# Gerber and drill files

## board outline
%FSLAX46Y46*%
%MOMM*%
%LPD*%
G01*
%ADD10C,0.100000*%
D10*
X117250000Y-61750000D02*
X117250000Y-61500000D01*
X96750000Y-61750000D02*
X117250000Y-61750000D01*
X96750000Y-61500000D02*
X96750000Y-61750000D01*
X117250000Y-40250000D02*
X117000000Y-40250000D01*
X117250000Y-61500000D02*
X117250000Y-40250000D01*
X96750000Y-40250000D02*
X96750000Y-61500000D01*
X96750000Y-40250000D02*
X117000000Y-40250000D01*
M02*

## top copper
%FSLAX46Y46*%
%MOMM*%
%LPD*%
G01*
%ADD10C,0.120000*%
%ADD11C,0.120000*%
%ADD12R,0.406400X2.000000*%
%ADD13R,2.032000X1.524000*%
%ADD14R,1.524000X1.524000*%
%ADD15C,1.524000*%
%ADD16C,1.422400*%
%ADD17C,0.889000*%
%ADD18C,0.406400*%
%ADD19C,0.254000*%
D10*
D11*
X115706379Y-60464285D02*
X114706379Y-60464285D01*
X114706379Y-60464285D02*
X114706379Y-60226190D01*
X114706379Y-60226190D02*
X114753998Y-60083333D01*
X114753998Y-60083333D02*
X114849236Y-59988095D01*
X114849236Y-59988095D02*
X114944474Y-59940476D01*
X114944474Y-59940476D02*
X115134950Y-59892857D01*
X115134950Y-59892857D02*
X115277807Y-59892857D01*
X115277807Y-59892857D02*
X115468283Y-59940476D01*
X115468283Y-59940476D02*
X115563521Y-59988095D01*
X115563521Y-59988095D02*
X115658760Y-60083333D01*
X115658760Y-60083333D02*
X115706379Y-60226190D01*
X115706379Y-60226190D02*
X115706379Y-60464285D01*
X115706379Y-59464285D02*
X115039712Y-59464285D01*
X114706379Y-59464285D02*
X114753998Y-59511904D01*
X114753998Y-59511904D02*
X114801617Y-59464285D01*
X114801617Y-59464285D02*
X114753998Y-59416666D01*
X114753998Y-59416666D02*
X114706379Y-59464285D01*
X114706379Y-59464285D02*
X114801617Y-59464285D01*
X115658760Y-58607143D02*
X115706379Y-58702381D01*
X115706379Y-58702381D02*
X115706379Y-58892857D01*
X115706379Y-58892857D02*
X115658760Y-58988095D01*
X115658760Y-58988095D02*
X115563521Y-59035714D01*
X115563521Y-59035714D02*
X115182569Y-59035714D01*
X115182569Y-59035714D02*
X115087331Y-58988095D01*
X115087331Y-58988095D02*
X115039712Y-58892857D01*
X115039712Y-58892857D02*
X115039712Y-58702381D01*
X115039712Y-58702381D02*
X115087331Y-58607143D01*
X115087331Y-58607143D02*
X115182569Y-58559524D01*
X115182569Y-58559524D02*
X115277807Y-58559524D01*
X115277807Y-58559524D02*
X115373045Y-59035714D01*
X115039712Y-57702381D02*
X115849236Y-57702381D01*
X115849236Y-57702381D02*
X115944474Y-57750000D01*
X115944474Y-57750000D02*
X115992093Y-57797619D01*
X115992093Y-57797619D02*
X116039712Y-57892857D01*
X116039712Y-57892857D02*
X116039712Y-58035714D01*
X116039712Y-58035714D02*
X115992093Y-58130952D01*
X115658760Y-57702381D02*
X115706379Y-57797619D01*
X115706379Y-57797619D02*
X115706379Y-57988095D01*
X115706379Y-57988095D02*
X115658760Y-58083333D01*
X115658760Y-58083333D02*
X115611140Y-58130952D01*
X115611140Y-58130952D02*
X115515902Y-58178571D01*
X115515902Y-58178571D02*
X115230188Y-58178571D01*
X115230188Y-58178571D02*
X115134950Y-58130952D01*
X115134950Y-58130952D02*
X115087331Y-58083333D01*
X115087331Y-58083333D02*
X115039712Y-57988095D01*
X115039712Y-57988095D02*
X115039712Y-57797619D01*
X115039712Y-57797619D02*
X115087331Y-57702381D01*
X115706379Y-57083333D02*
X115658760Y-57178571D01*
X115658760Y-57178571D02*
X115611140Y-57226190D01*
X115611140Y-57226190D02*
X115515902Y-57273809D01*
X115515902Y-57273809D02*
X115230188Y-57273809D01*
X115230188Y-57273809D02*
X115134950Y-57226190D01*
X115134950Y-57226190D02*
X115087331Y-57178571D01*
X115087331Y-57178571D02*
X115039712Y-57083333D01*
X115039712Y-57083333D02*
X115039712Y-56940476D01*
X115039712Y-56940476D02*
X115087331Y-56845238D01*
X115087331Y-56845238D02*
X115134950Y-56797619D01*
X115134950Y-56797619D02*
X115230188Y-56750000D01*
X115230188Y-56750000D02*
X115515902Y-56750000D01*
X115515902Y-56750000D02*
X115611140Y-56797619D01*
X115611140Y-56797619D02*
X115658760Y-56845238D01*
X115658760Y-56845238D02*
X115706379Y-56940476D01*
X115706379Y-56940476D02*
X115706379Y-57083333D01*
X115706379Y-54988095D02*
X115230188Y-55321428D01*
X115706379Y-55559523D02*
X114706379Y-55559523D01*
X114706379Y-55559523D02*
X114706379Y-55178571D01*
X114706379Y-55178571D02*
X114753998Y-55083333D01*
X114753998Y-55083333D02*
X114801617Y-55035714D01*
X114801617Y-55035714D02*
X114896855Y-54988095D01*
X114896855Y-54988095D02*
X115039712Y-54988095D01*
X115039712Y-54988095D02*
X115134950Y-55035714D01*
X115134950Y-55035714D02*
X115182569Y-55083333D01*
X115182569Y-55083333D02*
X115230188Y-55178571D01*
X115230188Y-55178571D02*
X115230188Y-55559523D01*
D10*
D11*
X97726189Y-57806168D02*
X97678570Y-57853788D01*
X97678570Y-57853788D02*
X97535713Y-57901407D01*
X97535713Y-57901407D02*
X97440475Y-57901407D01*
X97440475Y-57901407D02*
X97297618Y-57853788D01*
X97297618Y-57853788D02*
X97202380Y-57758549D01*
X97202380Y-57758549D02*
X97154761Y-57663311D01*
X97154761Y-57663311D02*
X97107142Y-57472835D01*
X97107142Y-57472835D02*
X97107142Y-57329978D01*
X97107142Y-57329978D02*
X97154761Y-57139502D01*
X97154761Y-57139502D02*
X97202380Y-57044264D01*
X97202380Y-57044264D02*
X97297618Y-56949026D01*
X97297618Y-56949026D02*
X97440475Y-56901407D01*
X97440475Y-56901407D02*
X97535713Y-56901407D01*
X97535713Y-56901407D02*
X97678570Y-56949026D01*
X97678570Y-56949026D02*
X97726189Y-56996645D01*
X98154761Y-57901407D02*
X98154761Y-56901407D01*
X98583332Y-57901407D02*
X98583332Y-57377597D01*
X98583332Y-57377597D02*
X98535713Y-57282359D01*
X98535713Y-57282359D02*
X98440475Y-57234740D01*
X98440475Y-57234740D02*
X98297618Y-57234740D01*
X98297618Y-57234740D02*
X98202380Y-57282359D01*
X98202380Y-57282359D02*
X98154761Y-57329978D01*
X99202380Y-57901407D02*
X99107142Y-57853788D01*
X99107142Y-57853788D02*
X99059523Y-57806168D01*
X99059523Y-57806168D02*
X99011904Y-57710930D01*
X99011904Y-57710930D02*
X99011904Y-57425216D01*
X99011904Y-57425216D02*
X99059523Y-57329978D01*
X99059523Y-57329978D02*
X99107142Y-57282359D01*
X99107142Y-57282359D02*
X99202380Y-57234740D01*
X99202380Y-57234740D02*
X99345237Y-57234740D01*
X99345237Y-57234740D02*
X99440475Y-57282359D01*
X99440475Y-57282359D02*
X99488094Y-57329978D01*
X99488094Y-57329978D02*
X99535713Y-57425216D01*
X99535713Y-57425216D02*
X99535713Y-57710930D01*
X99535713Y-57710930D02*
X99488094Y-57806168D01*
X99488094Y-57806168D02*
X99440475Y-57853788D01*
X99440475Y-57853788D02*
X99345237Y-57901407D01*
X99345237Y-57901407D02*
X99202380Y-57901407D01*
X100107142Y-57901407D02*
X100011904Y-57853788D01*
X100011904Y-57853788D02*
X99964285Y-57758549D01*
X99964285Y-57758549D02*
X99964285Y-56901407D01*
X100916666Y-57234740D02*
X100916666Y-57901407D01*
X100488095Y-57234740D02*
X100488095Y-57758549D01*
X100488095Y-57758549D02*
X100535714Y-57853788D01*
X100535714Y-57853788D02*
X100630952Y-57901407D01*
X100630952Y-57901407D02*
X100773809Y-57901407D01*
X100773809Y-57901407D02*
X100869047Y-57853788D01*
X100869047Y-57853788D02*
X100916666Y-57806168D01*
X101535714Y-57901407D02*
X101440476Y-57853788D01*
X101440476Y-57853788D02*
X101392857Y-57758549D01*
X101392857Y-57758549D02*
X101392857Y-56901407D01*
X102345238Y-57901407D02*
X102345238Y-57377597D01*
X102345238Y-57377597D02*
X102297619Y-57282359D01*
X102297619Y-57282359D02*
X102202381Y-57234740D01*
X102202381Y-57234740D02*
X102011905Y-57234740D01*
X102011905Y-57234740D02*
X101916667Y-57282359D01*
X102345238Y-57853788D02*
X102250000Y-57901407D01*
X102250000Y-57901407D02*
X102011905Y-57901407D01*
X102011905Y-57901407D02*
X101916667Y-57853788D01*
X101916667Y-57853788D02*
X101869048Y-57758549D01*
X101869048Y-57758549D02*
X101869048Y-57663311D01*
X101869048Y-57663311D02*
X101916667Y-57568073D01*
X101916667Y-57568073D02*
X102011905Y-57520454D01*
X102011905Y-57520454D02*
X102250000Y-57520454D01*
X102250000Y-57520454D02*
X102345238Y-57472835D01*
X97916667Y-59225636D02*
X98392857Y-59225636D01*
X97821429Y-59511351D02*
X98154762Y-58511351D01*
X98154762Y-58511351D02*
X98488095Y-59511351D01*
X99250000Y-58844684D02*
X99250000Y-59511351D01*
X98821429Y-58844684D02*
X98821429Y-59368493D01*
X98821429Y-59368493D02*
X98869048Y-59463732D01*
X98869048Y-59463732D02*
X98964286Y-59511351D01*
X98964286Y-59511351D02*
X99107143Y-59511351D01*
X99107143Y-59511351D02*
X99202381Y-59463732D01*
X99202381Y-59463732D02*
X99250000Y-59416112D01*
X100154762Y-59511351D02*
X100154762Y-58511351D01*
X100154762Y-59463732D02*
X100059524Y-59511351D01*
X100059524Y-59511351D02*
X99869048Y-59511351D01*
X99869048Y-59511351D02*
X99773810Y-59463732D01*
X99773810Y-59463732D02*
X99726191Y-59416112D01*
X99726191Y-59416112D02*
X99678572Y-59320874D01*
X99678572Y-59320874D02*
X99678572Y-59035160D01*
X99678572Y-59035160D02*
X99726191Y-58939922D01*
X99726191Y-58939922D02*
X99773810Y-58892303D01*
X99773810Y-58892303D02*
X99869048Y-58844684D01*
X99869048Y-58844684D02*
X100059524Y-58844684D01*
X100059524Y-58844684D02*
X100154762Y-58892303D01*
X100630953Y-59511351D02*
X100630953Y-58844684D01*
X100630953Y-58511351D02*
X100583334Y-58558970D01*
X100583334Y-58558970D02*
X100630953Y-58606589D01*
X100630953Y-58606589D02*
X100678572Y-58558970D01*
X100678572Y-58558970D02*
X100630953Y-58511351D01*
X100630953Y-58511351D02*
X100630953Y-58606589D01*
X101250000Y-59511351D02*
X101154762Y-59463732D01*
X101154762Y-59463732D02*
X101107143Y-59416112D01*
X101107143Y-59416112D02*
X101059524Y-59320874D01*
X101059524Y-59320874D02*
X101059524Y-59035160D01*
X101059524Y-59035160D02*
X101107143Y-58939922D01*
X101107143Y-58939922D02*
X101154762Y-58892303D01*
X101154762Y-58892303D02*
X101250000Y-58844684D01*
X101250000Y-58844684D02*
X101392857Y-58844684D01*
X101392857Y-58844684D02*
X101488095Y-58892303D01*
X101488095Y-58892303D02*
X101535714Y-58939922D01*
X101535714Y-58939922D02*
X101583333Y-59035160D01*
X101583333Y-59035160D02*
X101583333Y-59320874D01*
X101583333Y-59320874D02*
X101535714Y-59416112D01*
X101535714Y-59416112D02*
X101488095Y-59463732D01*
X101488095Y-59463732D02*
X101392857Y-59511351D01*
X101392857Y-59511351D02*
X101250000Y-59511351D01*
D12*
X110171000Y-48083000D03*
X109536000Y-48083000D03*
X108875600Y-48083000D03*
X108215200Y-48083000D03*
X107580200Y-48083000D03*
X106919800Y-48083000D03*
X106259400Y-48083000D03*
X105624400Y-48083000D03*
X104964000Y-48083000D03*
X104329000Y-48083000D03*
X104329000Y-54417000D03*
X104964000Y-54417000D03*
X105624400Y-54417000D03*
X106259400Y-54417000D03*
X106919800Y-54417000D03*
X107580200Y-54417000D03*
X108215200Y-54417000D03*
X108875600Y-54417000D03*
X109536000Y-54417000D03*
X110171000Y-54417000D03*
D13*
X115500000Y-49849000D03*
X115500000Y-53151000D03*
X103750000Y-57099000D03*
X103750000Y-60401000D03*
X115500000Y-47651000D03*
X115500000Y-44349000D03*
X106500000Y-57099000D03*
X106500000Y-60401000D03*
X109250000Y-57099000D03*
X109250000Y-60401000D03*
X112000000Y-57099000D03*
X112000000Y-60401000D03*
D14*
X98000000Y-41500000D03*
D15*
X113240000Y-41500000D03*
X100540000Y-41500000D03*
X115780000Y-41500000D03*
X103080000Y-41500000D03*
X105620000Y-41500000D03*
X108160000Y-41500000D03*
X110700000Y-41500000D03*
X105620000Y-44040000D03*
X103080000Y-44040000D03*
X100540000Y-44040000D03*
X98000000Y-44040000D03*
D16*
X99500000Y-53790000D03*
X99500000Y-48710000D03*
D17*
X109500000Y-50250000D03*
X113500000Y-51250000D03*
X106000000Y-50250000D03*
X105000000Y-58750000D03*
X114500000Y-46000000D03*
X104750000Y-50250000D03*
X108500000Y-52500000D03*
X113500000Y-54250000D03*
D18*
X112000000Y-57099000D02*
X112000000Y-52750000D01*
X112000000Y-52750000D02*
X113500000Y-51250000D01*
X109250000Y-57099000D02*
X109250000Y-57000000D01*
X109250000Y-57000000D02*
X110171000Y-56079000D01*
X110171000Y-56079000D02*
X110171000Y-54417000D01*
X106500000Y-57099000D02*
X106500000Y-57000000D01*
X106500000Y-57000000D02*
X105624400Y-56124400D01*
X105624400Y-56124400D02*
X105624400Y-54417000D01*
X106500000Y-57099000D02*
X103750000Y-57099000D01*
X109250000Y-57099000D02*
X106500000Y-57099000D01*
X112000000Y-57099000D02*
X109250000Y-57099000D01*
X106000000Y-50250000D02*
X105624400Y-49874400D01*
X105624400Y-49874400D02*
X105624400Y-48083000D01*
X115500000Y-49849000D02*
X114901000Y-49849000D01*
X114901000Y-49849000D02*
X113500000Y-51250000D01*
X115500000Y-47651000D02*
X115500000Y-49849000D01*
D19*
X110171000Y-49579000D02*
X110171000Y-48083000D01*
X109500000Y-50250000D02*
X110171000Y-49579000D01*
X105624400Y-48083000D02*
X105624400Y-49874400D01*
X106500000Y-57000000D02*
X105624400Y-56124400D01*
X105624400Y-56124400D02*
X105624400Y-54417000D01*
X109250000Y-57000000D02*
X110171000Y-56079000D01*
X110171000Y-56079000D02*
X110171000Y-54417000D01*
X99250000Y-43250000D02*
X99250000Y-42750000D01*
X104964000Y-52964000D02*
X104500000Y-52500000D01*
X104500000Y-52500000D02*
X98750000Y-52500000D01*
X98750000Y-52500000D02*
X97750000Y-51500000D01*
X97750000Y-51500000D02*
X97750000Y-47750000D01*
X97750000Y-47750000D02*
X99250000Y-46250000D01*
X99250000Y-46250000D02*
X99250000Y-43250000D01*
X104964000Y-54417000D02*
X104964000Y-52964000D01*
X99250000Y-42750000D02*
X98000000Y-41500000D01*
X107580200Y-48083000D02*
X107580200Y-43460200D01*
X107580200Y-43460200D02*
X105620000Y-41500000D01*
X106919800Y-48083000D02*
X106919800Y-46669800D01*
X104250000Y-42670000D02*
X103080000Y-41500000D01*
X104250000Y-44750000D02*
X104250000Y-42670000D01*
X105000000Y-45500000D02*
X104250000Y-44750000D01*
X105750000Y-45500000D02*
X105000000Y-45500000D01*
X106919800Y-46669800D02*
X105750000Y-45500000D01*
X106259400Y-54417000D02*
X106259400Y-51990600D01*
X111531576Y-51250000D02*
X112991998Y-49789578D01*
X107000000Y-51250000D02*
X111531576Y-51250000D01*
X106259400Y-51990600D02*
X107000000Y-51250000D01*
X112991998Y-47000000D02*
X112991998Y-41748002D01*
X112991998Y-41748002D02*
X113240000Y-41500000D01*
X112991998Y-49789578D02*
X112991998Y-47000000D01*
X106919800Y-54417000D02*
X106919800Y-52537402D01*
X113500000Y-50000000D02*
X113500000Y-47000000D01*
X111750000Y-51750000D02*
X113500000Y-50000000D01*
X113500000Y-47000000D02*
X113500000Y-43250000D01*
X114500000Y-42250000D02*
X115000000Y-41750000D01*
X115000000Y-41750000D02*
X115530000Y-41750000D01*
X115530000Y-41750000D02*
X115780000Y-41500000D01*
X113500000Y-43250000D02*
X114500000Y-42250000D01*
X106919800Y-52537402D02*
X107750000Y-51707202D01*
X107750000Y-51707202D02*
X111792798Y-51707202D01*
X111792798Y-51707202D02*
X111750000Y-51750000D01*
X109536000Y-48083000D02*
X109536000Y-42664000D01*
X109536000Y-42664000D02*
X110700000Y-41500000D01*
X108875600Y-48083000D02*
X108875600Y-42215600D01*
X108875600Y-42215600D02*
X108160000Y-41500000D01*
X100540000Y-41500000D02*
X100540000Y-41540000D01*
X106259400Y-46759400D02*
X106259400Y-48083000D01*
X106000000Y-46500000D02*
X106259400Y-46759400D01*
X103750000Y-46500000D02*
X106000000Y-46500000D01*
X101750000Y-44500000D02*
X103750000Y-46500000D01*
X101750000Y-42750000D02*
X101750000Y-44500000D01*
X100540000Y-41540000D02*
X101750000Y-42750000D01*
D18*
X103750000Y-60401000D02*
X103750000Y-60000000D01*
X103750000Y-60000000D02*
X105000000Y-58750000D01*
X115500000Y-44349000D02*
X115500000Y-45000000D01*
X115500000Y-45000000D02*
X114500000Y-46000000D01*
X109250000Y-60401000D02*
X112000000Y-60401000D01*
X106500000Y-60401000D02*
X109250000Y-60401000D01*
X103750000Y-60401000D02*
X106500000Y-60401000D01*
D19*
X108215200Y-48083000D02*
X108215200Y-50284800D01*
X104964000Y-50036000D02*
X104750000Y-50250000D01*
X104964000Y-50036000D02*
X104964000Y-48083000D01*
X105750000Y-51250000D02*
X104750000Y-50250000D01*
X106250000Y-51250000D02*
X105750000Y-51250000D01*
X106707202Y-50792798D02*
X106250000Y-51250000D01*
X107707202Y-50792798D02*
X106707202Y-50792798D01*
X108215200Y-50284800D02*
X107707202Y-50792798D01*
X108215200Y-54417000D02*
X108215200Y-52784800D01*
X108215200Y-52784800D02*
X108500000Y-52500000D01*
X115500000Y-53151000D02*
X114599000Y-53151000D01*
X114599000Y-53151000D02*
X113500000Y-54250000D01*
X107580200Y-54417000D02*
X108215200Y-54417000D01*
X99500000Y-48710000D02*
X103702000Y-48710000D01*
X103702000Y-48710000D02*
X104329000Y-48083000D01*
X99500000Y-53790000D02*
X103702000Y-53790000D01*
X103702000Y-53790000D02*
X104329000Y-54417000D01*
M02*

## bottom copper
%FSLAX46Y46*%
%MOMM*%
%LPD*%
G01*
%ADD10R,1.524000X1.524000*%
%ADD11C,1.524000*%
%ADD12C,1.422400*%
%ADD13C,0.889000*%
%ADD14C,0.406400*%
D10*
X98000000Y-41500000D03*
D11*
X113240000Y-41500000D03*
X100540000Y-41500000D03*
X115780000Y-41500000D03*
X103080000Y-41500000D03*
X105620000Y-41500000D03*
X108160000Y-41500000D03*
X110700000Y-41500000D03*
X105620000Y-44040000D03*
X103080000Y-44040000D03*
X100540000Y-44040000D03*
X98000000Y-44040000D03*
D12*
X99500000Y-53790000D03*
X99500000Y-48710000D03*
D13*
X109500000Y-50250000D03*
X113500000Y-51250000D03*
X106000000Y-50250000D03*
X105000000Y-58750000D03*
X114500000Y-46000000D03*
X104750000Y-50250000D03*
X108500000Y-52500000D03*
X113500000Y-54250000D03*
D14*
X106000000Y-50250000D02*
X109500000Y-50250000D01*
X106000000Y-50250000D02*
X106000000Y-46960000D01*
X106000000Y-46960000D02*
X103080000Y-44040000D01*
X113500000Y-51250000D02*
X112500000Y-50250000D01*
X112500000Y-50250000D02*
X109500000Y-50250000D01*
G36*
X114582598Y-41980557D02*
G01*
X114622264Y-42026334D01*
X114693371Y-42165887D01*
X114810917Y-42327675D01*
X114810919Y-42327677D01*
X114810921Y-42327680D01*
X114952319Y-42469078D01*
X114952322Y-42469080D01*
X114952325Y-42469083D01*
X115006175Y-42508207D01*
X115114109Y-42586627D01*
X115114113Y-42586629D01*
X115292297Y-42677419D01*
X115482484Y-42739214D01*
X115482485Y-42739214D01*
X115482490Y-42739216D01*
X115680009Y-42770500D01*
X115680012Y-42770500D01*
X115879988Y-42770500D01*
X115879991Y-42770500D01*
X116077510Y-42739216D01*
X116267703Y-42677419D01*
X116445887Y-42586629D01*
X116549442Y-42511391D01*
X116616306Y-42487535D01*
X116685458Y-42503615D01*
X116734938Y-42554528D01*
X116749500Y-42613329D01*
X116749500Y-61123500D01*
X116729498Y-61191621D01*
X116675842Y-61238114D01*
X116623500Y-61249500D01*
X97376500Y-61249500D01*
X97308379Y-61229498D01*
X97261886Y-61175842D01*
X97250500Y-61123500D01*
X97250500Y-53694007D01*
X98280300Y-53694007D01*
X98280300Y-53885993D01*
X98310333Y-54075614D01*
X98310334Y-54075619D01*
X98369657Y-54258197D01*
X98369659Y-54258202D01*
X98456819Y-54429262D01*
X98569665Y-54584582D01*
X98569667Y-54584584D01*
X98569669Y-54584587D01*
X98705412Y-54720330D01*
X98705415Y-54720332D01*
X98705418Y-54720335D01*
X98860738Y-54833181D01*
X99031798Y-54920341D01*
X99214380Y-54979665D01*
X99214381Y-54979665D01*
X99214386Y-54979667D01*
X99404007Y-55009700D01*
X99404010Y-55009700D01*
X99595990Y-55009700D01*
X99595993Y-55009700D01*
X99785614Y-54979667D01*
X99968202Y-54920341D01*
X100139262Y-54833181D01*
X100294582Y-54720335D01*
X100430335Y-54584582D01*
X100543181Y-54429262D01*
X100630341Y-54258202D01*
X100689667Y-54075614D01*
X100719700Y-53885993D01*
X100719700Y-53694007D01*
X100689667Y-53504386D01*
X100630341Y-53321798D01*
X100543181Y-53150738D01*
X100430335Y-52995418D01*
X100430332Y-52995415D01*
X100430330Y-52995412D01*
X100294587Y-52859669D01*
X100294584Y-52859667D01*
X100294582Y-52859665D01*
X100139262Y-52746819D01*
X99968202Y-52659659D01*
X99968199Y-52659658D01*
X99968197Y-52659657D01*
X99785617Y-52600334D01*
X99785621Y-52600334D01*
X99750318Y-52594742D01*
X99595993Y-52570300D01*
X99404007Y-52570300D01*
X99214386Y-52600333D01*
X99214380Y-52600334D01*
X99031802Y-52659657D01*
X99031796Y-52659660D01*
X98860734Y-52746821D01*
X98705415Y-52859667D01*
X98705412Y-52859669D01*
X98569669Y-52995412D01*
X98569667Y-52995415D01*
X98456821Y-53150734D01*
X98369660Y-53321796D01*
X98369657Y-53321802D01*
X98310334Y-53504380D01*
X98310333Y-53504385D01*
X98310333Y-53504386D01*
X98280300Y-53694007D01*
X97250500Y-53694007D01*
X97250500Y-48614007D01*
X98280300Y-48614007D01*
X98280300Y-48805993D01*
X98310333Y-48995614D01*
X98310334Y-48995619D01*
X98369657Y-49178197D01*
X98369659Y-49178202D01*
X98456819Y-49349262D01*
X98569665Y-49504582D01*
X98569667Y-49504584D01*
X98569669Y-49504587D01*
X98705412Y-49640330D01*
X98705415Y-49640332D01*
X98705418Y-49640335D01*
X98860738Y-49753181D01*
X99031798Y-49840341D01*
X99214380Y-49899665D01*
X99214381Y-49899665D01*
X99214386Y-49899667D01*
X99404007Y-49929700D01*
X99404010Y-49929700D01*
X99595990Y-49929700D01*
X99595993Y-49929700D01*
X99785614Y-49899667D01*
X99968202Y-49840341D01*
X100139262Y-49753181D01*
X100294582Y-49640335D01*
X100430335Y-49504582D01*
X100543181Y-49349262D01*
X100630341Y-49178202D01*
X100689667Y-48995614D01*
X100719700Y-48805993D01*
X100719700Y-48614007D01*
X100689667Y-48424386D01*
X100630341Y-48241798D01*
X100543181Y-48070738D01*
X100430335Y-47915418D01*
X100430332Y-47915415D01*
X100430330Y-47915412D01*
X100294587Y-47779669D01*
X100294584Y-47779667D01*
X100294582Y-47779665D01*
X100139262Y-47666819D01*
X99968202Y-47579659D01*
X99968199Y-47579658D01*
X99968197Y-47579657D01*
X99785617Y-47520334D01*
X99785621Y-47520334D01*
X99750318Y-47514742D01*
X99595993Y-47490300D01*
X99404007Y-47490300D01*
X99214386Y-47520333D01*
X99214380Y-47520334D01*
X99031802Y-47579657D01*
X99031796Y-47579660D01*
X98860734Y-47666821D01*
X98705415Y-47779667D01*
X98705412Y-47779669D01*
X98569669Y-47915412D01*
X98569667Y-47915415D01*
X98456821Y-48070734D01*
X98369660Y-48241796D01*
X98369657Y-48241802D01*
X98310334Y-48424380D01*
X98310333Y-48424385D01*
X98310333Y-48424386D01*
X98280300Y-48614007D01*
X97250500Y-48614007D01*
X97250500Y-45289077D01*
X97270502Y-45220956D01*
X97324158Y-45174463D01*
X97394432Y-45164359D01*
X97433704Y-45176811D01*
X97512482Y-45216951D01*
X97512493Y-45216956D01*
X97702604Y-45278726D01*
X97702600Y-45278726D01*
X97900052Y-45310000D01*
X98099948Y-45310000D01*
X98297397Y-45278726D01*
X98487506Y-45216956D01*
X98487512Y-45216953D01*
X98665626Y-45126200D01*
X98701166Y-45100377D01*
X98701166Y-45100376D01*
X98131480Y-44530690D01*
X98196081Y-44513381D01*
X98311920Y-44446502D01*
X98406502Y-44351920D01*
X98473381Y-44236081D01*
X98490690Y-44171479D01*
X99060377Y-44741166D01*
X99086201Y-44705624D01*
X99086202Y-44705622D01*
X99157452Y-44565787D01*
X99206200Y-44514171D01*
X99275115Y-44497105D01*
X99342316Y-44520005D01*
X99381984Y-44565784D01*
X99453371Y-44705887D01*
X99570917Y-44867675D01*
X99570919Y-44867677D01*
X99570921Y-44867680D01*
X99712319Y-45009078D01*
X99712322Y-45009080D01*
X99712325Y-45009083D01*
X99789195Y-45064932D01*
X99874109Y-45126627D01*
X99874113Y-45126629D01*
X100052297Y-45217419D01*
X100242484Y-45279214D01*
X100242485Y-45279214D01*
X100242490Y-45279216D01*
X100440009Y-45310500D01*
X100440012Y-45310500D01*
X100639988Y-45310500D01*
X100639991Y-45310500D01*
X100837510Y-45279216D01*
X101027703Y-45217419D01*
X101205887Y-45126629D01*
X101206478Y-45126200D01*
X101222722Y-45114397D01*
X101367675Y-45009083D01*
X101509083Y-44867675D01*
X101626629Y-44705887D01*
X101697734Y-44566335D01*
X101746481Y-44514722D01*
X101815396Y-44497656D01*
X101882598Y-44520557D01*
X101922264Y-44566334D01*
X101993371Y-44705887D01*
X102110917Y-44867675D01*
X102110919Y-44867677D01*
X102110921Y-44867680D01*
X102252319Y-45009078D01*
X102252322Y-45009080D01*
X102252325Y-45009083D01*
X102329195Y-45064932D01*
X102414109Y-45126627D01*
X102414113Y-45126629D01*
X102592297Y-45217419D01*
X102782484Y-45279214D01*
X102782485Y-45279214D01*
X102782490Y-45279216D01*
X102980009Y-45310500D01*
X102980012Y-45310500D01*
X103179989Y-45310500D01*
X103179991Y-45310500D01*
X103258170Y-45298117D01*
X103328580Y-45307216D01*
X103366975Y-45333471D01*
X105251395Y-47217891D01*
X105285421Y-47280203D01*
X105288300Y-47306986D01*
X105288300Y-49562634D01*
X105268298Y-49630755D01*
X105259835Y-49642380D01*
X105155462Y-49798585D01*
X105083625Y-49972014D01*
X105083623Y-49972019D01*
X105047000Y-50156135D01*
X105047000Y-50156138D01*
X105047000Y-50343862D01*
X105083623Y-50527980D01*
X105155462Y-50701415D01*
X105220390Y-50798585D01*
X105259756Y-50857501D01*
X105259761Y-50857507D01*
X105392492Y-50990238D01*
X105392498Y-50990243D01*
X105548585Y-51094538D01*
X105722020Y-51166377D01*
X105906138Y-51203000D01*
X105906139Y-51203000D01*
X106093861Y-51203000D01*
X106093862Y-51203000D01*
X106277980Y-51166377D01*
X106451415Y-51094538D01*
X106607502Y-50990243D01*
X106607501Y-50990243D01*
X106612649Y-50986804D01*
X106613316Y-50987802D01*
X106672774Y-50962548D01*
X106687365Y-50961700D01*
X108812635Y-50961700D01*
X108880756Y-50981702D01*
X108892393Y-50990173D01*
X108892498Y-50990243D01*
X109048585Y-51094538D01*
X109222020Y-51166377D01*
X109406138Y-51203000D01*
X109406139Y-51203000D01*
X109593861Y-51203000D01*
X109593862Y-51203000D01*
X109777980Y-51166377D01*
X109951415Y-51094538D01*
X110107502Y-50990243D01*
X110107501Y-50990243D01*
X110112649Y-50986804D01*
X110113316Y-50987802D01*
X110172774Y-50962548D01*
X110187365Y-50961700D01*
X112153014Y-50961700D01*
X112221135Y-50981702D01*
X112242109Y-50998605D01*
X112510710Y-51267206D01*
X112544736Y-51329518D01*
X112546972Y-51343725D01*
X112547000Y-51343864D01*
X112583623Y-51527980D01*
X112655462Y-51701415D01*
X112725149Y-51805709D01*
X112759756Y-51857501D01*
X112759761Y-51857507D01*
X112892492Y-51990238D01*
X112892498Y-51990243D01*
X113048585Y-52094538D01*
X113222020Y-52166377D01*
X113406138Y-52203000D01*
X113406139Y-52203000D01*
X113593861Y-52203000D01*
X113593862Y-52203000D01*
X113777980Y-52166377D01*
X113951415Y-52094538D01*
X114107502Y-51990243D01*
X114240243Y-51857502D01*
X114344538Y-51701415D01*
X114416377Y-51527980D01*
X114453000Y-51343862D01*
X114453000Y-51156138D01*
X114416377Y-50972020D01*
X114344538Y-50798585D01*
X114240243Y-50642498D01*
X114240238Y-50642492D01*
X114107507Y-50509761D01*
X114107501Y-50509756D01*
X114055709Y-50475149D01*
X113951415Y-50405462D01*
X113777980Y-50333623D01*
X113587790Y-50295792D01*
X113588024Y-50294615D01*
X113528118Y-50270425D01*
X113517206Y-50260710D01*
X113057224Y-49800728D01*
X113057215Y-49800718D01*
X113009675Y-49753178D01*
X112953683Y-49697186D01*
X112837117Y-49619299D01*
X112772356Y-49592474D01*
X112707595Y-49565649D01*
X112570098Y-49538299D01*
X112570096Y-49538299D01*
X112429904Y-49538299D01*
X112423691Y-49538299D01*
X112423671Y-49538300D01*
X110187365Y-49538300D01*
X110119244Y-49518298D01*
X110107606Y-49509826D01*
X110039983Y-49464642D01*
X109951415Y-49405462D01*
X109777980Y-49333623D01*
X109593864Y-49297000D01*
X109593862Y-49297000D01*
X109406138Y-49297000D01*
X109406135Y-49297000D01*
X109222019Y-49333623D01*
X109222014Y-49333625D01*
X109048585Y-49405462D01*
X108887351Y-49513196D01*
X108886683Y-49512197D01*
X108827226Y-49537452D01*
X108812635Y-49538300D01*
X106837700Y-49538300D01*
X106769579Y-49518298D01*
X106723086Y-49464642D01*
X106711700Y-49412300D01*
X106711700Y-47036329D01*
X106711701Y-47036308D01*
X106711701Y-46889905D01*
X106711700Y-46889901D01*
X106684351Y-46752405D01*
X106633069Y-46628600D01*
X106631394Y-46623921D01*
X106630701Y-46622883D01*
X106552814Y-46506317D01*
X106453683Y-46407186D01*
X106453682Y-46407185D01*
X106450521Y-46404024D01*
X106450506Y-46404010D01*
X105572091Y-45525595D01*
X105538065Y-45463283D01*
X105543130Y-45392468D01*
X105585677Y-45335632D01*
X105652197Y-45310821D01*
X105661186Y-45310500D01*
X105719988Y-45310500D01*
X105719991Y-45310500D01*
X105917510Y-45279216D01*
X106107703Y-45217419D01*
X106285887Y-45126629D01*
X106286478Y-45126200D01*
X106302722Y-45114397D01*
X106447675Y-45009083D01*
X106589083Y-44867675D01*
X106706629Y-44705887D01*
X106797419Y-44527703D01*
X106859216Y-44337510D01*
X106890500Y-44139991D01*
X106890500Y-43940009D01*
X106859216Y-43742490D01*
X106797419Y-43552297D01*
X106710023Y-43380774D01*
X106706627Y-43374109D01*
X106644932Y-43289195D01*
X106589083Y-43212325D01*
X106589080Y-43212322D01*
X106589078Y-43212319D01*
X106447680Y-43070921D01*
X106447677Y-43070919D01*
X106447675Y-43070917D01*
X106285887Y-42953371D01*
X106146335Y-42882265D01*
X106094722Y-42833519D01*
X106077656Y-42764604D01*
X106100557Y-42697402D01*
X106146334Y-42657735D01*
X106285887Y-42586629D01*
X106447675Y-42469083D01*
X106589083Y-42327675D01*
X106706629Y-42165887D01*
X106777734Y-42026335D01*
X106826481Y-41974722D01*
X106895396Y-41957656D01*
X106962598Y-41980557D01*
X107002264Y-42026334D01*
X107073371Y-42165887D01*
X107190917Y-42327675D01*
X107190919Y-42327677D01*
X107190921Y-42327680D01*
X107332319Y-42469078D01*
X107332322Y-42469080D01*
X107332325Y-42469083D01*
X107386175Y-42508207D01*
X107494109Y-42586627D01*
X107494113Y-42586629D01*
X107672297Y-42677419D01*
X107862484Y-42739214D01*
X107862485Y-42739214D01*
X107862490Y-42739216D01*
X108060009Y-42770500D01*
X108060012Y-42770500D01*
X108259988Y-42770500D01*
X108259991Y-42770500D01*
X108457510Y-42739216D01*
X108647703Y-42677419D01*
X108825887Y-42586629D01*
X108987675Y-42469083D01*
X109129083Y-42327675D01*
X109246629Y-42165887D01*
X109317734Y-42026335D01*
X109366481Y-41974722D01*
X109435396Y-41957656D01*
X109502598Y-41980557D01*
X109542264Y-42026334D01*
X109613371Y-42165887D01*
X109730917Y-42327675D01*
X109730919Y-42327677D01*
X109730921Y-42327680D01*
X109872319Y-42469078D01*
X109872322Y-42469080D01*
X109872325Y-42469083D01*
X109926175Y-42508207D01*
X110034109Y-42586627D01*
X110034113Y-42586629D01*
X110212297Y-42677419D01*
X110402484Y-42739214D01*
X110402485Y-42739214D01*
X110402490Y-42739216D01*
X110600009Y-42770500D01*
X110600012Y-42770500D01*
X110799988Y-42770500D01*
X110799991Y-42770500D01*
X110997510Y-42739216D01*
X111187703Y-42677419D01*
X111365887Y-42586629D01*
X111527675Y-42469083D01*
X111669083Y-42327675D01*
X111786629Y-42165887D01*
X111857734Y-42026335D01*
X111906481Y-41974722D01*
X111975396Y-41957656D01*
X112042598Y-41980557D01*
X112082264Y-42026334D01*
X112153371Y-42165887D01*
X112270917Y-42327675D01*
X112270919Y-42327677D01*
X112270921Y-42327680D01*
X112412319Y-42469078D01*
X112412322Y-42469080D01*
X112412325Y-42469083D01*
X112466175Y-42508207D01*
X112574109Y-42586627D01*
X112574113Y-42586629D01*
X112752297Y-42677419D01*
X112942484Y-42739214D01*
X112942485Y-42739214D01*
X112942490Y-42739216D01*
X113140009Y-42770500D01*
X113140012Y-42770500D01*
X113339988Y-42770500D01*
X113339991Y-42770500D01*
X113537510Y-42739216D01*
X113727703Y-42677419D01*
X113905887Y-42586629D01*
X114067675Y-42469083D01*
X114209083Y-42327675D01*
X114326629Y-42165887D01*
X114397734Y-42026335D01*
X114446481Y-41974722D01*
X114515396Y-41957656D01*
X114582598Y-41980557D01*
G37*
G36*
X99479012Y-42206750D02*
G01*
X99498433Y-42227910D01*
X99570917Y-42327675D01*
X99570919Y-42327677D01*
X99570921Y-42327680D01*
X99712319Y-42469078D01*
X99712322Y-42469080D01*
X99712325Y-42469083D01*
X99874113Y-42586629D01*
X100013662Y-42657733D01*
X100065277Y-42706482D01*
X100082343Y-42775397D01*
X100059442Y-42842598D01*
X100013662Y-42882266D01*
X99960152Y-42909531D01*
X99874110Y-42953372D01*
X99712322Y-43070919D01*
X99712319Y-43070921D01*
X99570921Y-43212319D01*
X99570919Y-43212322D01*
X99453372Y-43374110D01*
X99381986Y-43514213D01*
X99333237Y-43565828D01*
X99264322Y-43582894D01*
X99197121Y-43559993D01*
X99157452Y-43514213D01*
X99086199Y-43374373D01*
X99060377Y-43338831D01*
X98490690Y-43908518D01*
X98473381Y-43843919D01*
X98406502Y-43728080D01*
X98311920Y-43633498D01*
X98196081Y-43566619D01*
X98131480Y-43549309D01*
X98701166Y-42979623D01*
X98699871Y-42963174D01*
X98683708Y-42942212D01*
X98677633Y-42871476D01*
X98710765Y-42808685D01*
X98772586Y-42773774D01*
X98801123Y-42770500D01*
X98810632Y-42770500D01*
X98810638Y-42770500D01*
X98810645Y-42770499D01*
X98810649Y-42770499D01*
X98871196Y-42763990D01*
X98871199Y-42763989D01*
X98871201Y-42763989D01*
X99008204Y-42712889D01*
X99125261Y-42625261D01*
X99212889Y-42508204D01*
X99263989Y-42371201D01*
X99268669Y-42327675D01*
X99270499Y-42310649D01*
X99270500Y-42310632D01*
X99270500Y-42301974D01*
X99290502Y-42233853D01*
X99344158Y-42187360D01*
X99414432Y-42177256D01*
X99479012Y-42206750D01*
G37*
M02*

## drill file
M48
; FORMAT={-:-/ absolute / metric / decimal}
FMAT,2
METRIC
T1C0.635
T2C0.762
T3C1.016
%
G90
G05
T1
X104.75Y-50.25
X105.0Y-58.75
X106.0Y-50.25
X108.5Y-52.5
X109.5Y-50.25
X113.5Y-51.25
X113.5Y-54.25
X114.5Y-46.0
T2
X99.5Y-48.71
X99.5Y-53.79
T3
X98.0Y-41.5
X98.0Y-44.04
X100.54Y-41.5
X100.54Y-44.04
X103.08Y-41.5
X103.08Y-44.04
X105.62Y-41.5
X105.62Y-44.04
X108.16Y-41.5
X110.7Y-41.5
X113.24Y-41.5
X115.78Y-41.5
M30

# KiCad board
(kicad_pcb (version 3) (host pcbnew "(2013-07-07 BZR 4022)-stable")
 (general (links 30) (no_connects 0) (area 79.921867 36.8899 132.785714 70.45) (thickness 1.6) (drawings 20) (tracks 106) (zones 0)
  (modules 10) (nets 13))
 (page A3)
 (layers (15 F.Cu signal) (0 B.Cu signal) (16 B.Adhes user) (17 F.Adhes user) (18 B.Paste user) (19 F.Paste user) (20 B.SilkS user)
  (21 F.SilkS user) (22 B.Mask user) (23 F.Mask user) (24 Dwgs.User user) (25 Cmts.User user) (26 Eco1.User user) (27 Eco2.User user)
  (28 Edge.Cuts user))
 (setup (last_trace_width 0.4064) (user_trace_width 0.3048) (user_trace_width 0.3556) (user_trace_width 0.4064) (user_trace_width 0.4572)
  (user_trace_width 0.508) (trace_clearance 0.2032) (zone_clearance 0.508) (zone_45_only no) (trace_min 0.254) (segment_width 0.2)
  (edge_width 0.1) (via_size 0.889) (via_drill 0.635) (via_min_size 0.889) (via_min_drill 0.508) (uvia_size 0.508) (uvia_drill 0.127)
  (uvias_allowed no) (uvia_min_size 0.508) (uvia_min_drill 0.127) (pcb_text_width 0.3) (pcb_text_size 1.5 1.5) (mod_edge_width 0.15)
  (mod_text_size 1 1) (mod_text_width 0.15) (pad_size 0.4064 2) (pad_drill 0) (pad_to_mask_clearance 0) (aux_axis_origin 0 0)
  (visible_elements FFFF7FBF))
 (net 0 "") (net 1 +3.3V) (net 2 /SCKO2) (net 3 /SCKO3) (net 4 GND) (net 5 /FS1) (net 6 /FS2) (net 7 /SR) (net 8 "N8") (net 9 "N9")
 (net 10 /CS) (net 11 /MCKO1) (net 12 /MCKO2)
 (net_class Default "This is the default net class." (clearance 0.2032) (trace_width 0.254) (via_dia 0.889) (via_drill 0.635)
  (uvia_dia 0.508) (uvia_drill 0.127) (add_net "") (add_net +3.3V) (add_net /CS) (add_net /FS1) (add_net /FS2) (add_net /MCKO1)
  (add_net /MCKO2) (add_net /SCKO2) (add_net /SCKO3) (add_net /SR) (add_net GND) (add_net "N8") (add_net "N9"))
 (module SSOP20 (layer F.Cu) (at 107.25 51.25 180)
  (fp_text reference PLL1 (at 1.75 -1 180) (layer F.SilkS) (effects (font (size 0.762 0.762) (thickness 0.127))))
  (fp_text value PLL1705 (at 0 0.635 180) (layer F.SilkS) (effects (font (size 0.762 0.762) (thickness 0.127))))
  (pad 1 smd rect (at -2.921 3.167 180) (size 0.4064 2) (layers F.Cu F.Paste F.Mask) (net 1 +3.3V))
  (pad 2 smd rect (at -2.286 3.167 180) (size 0.4064 2) (layers F.Cu F.Paste F.Mask) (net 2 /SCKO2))
  (pad 3 smd rect (at -1.6256 3.167 180) (size 0.4064 2) (layers F.Cu F.Paste F.Mask) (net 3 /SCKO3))
  (pad 4 smd rect (at -0.9652 3.167 180) (size 0.4064 2) (layers F.Cu F.Paste F.Mask) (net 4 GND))
  (pad 5 smd rect (at -0.3302 3.167 180) (size 0.4064 2) (layers F.Cu F.Paste F.Mask) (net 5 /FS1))
  (pad 6 smd rect (at 0.3302 3.167 180) (size 0.4064 2) (layers F.Cu F.Paste F.Mask) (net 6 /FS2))
  (pad 7 smd rect (at 0.9906 3.167 180) (size 0.4064 2) (layers F.Cu F.Paste F.Mask) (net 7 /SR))
  (pad 8 smd rect (at 1.6256 3.167 180) (size 0.4064 2) (layers F.Cu F.Paste F.Mask) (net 1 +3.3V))
  (pad 9 smd rect (at 2.286 3.167 180) (size 0.4064 2) (layers F.Cu F.Paste F.Mask) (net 4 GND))
  (pad 10 smd rect (at 2.921 3.167 180) (size 0.4064 2) (layers F.Cu F.Paste F.Mask) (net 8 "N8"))
  (pad 11 smd rect (at 2.921 -3.167 180) (size 0.4064 2) (layers F.Cu F.Paste F.Mask) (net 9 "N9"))
  (pad 12 smd rect (at 2.286 -3.167 180) (size 0.4064 2) (layers F.Cu F.Paste F.Mask) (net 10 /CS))
  (pad 13 smd rect (at 1.6256 -3.167 180) (size 0.4064 2) (layers F.Cu F.Paste F.Mask) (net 1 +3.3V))
  (pad 14 smd rect (at 0.9906 -3.167 180) (size 0.4064 2) (layers F.Cu F.Paste F.Mask) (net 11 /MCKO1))
  (pad 15 smd rect (at 0.3302 -3.167 180) (size 0.4064 2) (layers F.Cu F.Paste F.Mask) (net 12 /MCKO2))
  (pad 16 smd rect (at -0.3302 -3.167 180) (size 0.4064 2) (layers F.Cu F.Paste F.Mask) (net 4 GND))
  (pad 17 smd rect (at -0.9652 -3.167 180) (size 0.4064 2) (layers F.Cu F.Paste F.Mask) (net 4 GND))
  (pad 18 smd rect (at -1.6256 -3.167 180) (size 0.4064 2) (layers F.Cu F.Paste F.Mask))
  (pad 19 smd rect (at -2.286 -3.167 180) (size 0.4064 2) (layers F.Cu F.Paste F.Mask))
  (pad 20 smd rect (at -2.921 -3.167 180) (size 0.4064 2) (layers F.Cu F.Paste F.Mask) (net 1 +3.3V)))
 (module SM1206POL (layer F.Cu) (at 115.5 51.5 270)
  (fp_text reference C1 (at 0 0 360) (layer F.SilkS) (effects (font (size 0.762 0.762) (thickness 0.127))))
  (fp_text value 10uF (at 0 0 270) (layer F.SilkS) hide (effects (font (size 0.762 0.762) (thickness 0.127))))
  (pad 1 smd rect (at -1.651 0 270) (size 1.524 2.032) (layers F.Cu F.Paste F.Mask) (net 1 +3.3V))
  (pad 2 smd rect (at 1.651 0 270) (size 1.524 2.032) (layers F.Cu F.Paste F.Mask) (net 4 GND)))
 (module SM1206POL (layer F.Cu) (at 103.75 58.75 270)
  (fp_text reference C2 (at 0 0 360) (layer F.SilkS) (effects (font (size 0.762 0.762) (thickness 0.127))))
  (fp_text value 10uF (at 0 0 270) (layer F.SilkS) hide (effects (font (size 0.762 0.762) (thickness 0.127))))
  (pad 1 smd rect (at -1.651 0 270) (size 1.524 2.032) (layers F.Cu F.Paste F.Mask) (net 1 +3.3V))
  (pad 2 smd rect (at 1.651 0 270) (size 1.524 2.032) (layers F.Cu F.Paste F.Mask) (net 4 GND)))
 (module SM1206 (layer F.Cu) (at 115.5 46 90)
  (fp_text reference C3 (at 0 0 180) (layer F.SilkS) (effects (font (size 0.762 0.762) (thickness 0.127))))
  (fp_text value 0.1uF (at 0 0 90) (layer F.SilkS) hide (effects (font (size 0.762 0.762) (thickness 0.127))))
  (pad 1 smd rect (at -1.651 0 90) (size 1.524 2.032) (layers F.Cu F.Paste F.Mask) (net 1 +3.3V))
  (pad 2 smd rect (at 1.651 0 90) (size 1.524 2.032) (layers F.Cu F.Paste F.Mask) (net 4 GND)))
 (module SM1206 (layer F.Cu) (at 106.5 58.75 270)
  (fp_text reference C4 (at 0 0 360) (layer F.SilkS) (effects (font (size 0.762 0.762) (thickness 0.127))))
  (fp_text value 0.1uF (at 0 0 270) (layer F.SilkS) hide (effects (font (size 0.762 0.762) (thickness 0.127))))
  (pad 1 smd rect (at -1.651 0 270) (size 1.524 2.032) (layers F.Cu F.Paste F.Mask) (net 1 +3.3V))
  (pad 2 smd rect (at 1.651 0 270) (size 1.524 2.032) (layers F.Cu F.Paste F.Mask) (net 4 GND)))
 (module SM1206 (layer F.Cu) (at 109.25 58.75 270)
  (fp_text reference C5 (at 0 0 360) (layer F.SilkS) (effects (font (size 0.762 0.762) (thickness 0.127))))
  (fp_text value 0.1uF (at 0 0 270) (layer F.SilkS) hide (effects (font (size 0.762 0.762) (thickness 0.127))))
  (pad 1 smd rect (at -1.651 0 270) (size 1.524 2.032) (layers F.Cu F.Paste F.Mask) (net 1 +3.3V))
  (pad 2 smd rect (at 1.651 0 270) (size 1.524 2.032) (layers F.Cu F.Paste F.Mask) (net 4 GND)))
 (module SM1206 (layer F.Cu) (at 112 58.75 270)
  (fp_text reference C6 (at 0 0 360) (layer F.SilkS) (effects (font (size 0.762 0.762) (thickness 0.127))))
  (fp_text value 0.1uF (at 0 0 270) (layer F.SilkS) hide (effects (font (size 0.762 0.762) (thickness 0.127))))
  (pad 1 smd rect (at -1.651 0 270) (size 1.524 2.032) (layers F.Cu F.Paste F.Mask) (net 1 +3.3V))
  (pad 2 smd rect (at 1.651 0 270) (size 1.524 2.032) (layers F.Cu F.Paste F.Mask) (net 4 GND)))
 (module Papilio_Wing (layer F.Cu) (at 98 41.5)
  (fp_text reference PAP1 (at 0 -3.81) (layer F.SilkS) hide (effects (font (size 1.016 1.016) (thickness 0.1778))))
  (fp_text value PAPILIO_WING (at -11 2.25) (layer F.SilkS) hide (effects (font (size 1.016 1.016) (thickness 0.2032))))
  (pad 1 thru_hole rect (at 0 0) (size 1.524 1.524) (drill 1.016) (layers *.Cu *.Mask F.SilkS) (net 10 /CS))
  (pad 7 thru_hole circle (at 15.24 0) (size 1.524 1.524) (drill 1.016) (layers *.Cu *.Mask F.SilkS) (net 11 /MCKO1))
  (pad 2 thru_hole circle (at 2.54 0) (size 1.524 1.524) (drill 1.016) (layers *.Cu *.Mask F.SilkS) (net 7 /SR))
  (pad 8 thru_hole circle (at 17.78 0) (size 1.524 1.524) (drill 1.016) (layers *.Cu *.Mask F.SilkS) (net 12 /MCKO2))
  (pad 3 thru_hole circle (at 5.08 0) (size 1.524 1.524) (drill 1.016) (layers *.Cu *.Mask F.SilkS) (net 6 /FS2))
  (pad 4 thru_hole circle (at 7.62 0) (size 1.524 1.524) (drill 1.016) (layers *.Cu *.Mask F.SilkS) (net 5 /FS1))
  (pad 5 thru_hole circle (at 10.16 0) (size 1.524 1.524) (drill 1.016) (layers *.Cu *.Mask F.SilkS) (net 3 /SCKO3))
  (pad 6 thru_hole circle (at 12.7 0) (size 1.524 1.524) (drill 1.016) (layers *.Cu *.Mask F.SilkS) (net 2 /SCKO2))
  (pad 9 thru_hole circle (at 7.62 2.54) (size 1.524 1.524) (drill 1.016) (layers *.Cu *.Mask F.SilkS))
  (pad 10 thru_hole circle (at 5.08 2.54) (size 1.524 1.524) (drill 1.016) (layers *.Cu *.Mask F.SilkS) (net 1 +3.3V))
  (pad 11 thru_hole circle (at 2.54 2.54) (size 1.524 1.524) (drill 1.016) (layers *.Cu *.Mask F.SilkS))
  (pad 12 thru_hole circle (at 0 2.54) (size 1.524 1.524) (drill 1.016) (layers *.Cu *.Mask F.SilkS) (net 4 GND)))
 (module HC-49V (layer F.Cu) (at 99.5 51.25 90) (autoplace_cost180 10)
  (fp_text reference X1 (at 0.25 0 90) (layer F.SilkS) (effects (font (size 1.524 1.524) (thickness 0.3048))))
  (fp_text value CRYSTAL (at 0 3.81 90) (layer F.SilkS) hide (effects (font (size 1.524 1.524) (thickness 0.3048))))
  (pad 1 thru_hole circle (at -2.54 0 90) (size 1.4224 1.4224) (drill 0.762) (layers *.Cu *.Mask F.SilkS) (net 9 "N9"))
  (pad 2 thru_hole circle (at 2.54 0 90) (size 1.4224 1.4224) (drill 0.762) (layers *.Cu *.Mask F.SilkS) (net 8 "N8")))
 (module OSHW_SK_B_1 (layer F.Cu) (at 105.75 55.5)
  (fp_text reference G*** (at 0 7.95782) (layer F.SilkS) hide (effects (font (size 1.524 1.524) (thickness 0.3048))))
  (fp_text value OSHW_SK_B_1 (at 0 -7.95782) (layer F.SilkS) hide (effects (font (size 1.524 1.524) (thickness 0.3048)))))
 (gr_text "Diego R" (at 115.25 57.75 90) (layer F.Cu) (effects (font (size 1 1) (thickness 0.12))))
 (gr_line (start 117.25 61.75) (end 117.25 61.5) (angle 90) (layer Edge.Cuts) (width 0.1))
 (gr_line (start 96.75 61.75) (end 117.25 61.75) (angle 90) (layer Edge.Cuts) (width 0.1))
 (gr_line (start 96.75 61.5) (end 96.75 61.75) (angle 90) (layer Edge.Cuts) (width 0.1))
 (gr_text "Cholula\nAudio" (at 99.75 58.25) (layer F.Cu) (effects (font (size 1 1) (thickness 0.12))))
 (gr_line (start 117.25 40.25) (end 117 40.25) (angle 90) (layer Edge.Cuts) (width 0.1))
 (gr_line (start 117.25 61.5) (end 117.25 40.25) (angle 90) (layer Edge.Cuts) (width 0.1))
 (gr_line (start 96.75 40.25) (end 96.75 61.5) (angle 90) (layer Edge.Cuts) (width 0.1))
 (gr_line (start 96.75 40.25) (end 117 40.25) (angle 90) (layer Edge.Cuts) (width 0.1))
 (segment (start 106 50.25) (end 109.5 50.25) (width 0.4064) (layer B.Cu) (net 1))
 (segment (start 112 57.099) (end 112 52.75) (width 0.4064) (layer F.Cu) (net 1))
 (segment (start 112 52.75) (end 113.5 51.25) (width 0.4064) (layer F.Cu) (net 1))
 (segment (start 109.25 57.099) (end 109.25 57) (width 0.4064) (layer F.Cu) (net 1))
 (segment (start 109.25 57) (end 110.171 56.079) (width 0.4064) (layer F.Cu) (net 1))
 (segment (start 110.171 56.079) (end 110.171 54.417) (width 0.4064) (layer F.Cu) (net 1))
 (segment (start 106.5 57.099) (end 106.5 57) (width 0.4064) (layer F.Cu) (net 1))
 (segment (start 106.5 57) (end 105.6244 56.1244) (width 0.4064) (layer F.Cu) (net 1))
 (segment (start 105.6244 56.1244) (end 105.6244 54.417) (width 0.4064) (layer F.Cu) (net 1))
 (segment (start 106.5 57.099) (end 103.75 57.099) (width 0.4064) (layer F.Cu) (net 1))
 (segment (start 109.25 57.099) (end 106.5 57.099) (width 0.4064) (layer F.Cu) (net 1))
 (segment (start 112 57.099) (end 109.25 57.099) (width 0.4064) (layer F.Cu) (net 1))
 (segment (start 106 50.25) (end 106 46.96) (width 0.4064) (layer B.Cu) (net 1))
 (segment (start 106 46.96) (end 103.08 44.04) (width 0.4064) (layer B.Cu) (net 1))
 (segment (start 106 50.25) (end 105.6244 49.8744) (width 0.4064) (layer F.Cu) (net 1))
 (segment (start 105.6244 49.8744) (end 105.6244 48.083) (width 0.4064) (layer F.Cu) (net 1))
 (segment (start 115.5 49.849) (end 114.901 49.849) (width 0.4064) (layer F.Cu) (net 1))
 (segment (start 114.901 49.849) (end 113.5 51.25) (width 0.4064) (layer F.Cu) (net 1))
 (via (at 109.5 50.25) (size 0.889) (layers F.Cu B.Cu) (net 1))
 (via (at 113.5 51.25) (size 0.889) (layers F.Cu B.Cu) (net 1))
 (segment (start 113.5 51.25) (end 112.5 50.25) (width 0.4064) (layer B.Cu) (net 1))
 (segment (start 112.5 50.25) (end 109.5 50.25) (width 0.4064) (layer B.Cu) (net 1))
 (segment (start 115.5 47.651) (end 115.5 49.849) (width 0.4064) (layer F.Cu) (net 1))
 (segment (start 110.171 49.579) (end 110.171 48.083) (width 0.254) (layer F.Cu) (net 1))
 (segment (start 109.5 50.25) (end 110.171 49.579) (width 0.254) (layer F.Cu) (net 1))
 (segment (start 105.6244 48.083) (end 105.6244 49.8744) (width 0.254) (layer F.Cu) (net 1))
 (via (at 106 50.25) (size 0.889) (layers F.Cu B.Cu) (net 1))
 (segment (start 106.5 57) (end 105.6244 56.1244) (width 0.254) (layer F.Cu) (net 1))
 (segment (start 105.6244 56.1244) (end 105.6244 54.417) (width 0.254) (layer F.Cu) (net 1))
 (segment (start 109.25 57) (end 110.171 56.079) (width 0.254) (layer F.Cu) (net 1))
 (segment (start 110.171 56.079) (end 110.171 54.417) (width 0.254) (layer F.Cu) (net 1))
 (segment (start 99.25 43.25) (end 99.25 42.75) (width 0.254) (layer F.Cu) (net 10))
 (segment (start 104.964 52.964) (end 104.5 52.5) (width 0.254) (layer F.Cu) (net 10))
 (segment (start 104.5 52.5) (end 98.75 52.5) (width 0.254) (layer F.Cu) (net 10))
 (segment (start 98.75 52.5) (end 97.75 51.5) (width 0.254) (layer F.Cu) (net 10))
 (segment (start 97.75 51.5) (end 97.75 47.75) (width 0.254) (layer F.Cu) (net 10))
 (segment (start 97.75 47.75) (end 99.25 46.25) (width 0.254) (layer F.Cu) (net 10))
 (segment (start 99.25 46.25) (end 99.25 43.25) (width 0.254) (layer F.Cu) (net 10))
 (segment (start 104.964 54.417) (end 104.964 52.964) (width 0.254) (layer F.Cu) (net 10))
 (segment (start 99.25 42.75) (end 98 41.5) (width 0.254) (layer F.Cu) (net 10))
 (segment (start 107.5802 48.083) (end 107.5802 43.4602) (width 0.254) (layer F.Cu) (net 5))
 (segment (start 107.5802 43.4602) (end 105.62 41.5) (width 0.254) (layer F.Cu) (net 5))
 (segment (start 106.9198 48.083) (end 106.9198 46.6698) (width 0.254) (layer F.Cu) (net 6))
 (segment (start 104.25 42.67) (end 103.08 41.5) (width 0.254) (layer F.Cu) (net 6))
 (segment (start 104.25 44.75) (end 104.25 42.67) (width 0.254) (layer F.Cu) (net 6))
 (segment (start 105 45.5) (end 104.25 44.75) (width 0.254) (layer F.Cu) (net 6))
 (segment (start 105.75 45.5) (end 105 45.5) (width 0.254) (layer F.Cu) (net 6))
 (segment (start 106.9198 46.6698) (end 105.75 45.5) (width 0.254) (layer F.Cu) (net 6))
 (segment (start 106.2594 54.417) (end 106.2594 51.9906) (width 0.254) (layer F.Cu) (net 11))
 (segment (start 111.531576 51.25) (end 112.991998 49.789578) (width 0.254) (layer F.Cu) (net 11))
 (segment (start 107 51.25) (end 111.531576 51.25) (width 0.254) (layer F.Cu) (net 11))
 (segment (start 106.2594 51.9906) (end 107 51.25) (width 0.254) (layer F.Cu) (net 11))
 (segment (start 112.991998 47) (end 112.991998 41.748002) (width 0.254) (layer F.Cu) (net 11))
 (segment (start 112.991998 41.748002) (end 113.24 41.5) (width 0.254) (layer F.Cu) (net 11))
 (segment (start 112.991998 49.789578) (end 112.991998 47) (width 0.254) (layer F.Cu) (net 11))
 (segment (start 106.9198 54.417) (end 106.9198 52.537402) (width 0.254) (layer F.Cu) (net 12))
 (segment (start 113.5 50) (end 113.5 47) (width 0.254) (layer F.Cu) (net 12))
 (segment (start 111.75 51.75) (end 113.5 50) (width 0.254) (layer F.Cu) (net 12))
 (segment (start 113.5 47) (end 113.5 43.25) (width 0.254) (layer F.Cu) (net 12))
 (segment (start 114.5 42.25) (end 115 41.75) (width 0.254) (layer F.Cu) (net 12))
 (segment (start 115 41.75) (end 115.53 41.75) (width 0.254) (layer F.Cu) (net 12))
 (segment (start 115.53 41.75) (end 115.78 41.5) (width 0.254) (layer F.Cu) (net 12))
 (segment (start 113.5 43.25) (end 114.5 42.25) (width 0.254) (layer F.Cu) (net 12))
 (segment (start 106.9198 52.537402) (end 107.75 51.707202) (width 0.254) (layer F.Cu) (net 12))
 (segment (start 107.75 51.707202) (end 111.792798 51.707202) (width 0.254) (layer F.Cu) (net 12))
 (segment (start 111.792798 51.707202) (end 111.75 51.75) (width 0.254) (layer F.Cu) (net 12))
 (segment (start 109.536 48.083) (end 109.536 42.664) (width 0.254) (layer F.Cu) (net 2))
 (segment (start 109.536 42.664) (end 110.7 41.5) (width 0.254) (layer F.Cu) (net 2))
 (segment (start 108.8756 48.083) (end 108.8756 42.2156) (width 0.254) (layer F.Cu) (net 3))
 (segment (start 108.8756 42.2156) (end 108.16 41.5) (width 0.254) (layer F.Cu) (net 3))
 (segment (start 100.54 41.5) (end 100.54 41.54) (width 0.254) (layer F.Cu) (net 7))
 (segment (start 106.2594 46.7594) (end 106.2594 48.083) (width 0.254) (layer F.Cu) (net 7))
 (segment (start 106 46.5) (end 106.2594 46.7594) (width 0.254) (layer F.Cu) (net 7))
 (segment (start 103.75 46.5) (end 106 46.5) (width 0.254) (layer F.Cu) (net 7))
 (segment (start 101.75 44.5) (end 103.75 46.5) (width 0.254) (layer F.Cu) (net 7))
 (segment (start 101.75 42.75) (end 101.75 44.5) (width 0.254) (layer F.Cu) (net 7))
 (segment (start 100.54 41.54) (end 101.75 42.75) (width 0.254) (layer F.Cu) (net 7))
 (segment (start 103.75 60.401) (end 103.75 60) (width 0.4064) (layer F.Cu) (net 4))
 (via (at 105 58.75) (size 0.889) (layers F.Cu B.Cu) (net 4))
 (segment (start 103.75 60) (end 105 58.75) (width 0.4064) (layer F.Cu) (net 4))
 (segment (start 115.5 44.349) (end 115.5 45) (width 0.4064) (layer F.Cu) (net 4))
 (via (at 114.5 46) (size 0.889) (layers F.Cu B.Cu) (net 4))
 (segment (start 115.5 45) (end 114.5 46) (width 0.4064) (layer F.Cu) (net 4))
 (segment (start 109.25 60.401) (end 112 60.401) (width 0.4064) (layer F.Cu) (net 4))
 (segment (start 106.5 60.401) (end 109.25 60.401) (width 0.4064) (layer F.Cu) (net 4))
 (segment (start 103.75 60.401) (end 106.5 60.401) (width 0.4064) (layer F.Cu) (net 4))
 (segment (start 108.2152 48.083) (end 108.2152 50.2848) (width 0.254) (layer F.Cu) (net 4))
 (segment (start 104.964 50.036) (end 104.75 50.25) (width 0.254) (layer F.Cu) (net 4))
 (via (at 104.75 50.25) (size 0.889) (layers F.Cu B.Cu) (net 4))
 (segment (start 104.964 50.036) (end 104.964 48.083) (width 0.254) (layer F.Cu) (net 4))
 (segment (start 105.75 51.25) (end 104.75 50.25) (width 0.254) (layer F.Cu) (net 4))
 (segment (start 106.25 51.25) (end 105.75 51.25) (width 0.254) (layer F.Cu) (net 4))
 (segment (start 106.707202 50.792798) (end 106.25 51.25) (width 0.254) (layer F.Cu) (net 4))
 (segment (start 107.707202 50.792798) (end 106.707202 50.792798) (width 0.254) (layer F.Cu) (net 4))
 (segment (start 108.2152 50.2848) (end 107.707202 50.792798) (width 0.254) (layer F.Cu) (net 4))
 (segment (start 108.2152 54.417) (end 108.2152 52.7848) (width 0.254) (layer F.Cu) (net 4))
 (via (at 108.5 52.5) (size 0.889) (layers F.Cu B.Cu) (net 4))
 (segment (start 108.2152 52.7848) (end 108.5 52.5) (width 0.254) (layer F.Cu) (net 4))
 (segment (start 115.5 53.151) (end 114.599 53.151) (width 0.254) (layer F.Cu) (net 4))
 (via (at 113.5 54.25) (size 0.889) (layers F.Cu B.Cu) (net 4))
 (segment (start 114.599 53.151) (end 113.5 54.25) (width 0.254) (layer F.Cu) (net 4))
 (segment (start 107.5802 54.417) (end 108.2152 54.417) (width 0.254) (layer F.Cu) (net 4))
 (segment (start 99.5 48.71) (end 103.702 48.71) (width 0.254) (layer F.Cu) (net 8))
 (segment (start 103.702 48.71) (end 104.329 48.083) (width 0.254) (layer F.Cu) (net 8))
 (segment (start 99.5 53.79) (end 103.702 53.79) (width 0.254) (layer F.Cu) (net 9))
 (segment (start 103.702 53.79) (end 104.329 54.417) (width 0.254) (layer F.Cu) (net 9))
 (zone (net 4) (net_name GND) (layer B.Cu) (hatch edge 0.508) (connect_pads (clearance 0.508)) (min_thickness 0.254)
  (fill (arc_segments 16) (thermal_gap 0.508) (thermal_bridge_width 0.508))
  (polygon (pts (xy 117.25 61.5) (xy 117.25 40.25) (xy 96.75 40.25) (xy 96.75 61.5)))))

